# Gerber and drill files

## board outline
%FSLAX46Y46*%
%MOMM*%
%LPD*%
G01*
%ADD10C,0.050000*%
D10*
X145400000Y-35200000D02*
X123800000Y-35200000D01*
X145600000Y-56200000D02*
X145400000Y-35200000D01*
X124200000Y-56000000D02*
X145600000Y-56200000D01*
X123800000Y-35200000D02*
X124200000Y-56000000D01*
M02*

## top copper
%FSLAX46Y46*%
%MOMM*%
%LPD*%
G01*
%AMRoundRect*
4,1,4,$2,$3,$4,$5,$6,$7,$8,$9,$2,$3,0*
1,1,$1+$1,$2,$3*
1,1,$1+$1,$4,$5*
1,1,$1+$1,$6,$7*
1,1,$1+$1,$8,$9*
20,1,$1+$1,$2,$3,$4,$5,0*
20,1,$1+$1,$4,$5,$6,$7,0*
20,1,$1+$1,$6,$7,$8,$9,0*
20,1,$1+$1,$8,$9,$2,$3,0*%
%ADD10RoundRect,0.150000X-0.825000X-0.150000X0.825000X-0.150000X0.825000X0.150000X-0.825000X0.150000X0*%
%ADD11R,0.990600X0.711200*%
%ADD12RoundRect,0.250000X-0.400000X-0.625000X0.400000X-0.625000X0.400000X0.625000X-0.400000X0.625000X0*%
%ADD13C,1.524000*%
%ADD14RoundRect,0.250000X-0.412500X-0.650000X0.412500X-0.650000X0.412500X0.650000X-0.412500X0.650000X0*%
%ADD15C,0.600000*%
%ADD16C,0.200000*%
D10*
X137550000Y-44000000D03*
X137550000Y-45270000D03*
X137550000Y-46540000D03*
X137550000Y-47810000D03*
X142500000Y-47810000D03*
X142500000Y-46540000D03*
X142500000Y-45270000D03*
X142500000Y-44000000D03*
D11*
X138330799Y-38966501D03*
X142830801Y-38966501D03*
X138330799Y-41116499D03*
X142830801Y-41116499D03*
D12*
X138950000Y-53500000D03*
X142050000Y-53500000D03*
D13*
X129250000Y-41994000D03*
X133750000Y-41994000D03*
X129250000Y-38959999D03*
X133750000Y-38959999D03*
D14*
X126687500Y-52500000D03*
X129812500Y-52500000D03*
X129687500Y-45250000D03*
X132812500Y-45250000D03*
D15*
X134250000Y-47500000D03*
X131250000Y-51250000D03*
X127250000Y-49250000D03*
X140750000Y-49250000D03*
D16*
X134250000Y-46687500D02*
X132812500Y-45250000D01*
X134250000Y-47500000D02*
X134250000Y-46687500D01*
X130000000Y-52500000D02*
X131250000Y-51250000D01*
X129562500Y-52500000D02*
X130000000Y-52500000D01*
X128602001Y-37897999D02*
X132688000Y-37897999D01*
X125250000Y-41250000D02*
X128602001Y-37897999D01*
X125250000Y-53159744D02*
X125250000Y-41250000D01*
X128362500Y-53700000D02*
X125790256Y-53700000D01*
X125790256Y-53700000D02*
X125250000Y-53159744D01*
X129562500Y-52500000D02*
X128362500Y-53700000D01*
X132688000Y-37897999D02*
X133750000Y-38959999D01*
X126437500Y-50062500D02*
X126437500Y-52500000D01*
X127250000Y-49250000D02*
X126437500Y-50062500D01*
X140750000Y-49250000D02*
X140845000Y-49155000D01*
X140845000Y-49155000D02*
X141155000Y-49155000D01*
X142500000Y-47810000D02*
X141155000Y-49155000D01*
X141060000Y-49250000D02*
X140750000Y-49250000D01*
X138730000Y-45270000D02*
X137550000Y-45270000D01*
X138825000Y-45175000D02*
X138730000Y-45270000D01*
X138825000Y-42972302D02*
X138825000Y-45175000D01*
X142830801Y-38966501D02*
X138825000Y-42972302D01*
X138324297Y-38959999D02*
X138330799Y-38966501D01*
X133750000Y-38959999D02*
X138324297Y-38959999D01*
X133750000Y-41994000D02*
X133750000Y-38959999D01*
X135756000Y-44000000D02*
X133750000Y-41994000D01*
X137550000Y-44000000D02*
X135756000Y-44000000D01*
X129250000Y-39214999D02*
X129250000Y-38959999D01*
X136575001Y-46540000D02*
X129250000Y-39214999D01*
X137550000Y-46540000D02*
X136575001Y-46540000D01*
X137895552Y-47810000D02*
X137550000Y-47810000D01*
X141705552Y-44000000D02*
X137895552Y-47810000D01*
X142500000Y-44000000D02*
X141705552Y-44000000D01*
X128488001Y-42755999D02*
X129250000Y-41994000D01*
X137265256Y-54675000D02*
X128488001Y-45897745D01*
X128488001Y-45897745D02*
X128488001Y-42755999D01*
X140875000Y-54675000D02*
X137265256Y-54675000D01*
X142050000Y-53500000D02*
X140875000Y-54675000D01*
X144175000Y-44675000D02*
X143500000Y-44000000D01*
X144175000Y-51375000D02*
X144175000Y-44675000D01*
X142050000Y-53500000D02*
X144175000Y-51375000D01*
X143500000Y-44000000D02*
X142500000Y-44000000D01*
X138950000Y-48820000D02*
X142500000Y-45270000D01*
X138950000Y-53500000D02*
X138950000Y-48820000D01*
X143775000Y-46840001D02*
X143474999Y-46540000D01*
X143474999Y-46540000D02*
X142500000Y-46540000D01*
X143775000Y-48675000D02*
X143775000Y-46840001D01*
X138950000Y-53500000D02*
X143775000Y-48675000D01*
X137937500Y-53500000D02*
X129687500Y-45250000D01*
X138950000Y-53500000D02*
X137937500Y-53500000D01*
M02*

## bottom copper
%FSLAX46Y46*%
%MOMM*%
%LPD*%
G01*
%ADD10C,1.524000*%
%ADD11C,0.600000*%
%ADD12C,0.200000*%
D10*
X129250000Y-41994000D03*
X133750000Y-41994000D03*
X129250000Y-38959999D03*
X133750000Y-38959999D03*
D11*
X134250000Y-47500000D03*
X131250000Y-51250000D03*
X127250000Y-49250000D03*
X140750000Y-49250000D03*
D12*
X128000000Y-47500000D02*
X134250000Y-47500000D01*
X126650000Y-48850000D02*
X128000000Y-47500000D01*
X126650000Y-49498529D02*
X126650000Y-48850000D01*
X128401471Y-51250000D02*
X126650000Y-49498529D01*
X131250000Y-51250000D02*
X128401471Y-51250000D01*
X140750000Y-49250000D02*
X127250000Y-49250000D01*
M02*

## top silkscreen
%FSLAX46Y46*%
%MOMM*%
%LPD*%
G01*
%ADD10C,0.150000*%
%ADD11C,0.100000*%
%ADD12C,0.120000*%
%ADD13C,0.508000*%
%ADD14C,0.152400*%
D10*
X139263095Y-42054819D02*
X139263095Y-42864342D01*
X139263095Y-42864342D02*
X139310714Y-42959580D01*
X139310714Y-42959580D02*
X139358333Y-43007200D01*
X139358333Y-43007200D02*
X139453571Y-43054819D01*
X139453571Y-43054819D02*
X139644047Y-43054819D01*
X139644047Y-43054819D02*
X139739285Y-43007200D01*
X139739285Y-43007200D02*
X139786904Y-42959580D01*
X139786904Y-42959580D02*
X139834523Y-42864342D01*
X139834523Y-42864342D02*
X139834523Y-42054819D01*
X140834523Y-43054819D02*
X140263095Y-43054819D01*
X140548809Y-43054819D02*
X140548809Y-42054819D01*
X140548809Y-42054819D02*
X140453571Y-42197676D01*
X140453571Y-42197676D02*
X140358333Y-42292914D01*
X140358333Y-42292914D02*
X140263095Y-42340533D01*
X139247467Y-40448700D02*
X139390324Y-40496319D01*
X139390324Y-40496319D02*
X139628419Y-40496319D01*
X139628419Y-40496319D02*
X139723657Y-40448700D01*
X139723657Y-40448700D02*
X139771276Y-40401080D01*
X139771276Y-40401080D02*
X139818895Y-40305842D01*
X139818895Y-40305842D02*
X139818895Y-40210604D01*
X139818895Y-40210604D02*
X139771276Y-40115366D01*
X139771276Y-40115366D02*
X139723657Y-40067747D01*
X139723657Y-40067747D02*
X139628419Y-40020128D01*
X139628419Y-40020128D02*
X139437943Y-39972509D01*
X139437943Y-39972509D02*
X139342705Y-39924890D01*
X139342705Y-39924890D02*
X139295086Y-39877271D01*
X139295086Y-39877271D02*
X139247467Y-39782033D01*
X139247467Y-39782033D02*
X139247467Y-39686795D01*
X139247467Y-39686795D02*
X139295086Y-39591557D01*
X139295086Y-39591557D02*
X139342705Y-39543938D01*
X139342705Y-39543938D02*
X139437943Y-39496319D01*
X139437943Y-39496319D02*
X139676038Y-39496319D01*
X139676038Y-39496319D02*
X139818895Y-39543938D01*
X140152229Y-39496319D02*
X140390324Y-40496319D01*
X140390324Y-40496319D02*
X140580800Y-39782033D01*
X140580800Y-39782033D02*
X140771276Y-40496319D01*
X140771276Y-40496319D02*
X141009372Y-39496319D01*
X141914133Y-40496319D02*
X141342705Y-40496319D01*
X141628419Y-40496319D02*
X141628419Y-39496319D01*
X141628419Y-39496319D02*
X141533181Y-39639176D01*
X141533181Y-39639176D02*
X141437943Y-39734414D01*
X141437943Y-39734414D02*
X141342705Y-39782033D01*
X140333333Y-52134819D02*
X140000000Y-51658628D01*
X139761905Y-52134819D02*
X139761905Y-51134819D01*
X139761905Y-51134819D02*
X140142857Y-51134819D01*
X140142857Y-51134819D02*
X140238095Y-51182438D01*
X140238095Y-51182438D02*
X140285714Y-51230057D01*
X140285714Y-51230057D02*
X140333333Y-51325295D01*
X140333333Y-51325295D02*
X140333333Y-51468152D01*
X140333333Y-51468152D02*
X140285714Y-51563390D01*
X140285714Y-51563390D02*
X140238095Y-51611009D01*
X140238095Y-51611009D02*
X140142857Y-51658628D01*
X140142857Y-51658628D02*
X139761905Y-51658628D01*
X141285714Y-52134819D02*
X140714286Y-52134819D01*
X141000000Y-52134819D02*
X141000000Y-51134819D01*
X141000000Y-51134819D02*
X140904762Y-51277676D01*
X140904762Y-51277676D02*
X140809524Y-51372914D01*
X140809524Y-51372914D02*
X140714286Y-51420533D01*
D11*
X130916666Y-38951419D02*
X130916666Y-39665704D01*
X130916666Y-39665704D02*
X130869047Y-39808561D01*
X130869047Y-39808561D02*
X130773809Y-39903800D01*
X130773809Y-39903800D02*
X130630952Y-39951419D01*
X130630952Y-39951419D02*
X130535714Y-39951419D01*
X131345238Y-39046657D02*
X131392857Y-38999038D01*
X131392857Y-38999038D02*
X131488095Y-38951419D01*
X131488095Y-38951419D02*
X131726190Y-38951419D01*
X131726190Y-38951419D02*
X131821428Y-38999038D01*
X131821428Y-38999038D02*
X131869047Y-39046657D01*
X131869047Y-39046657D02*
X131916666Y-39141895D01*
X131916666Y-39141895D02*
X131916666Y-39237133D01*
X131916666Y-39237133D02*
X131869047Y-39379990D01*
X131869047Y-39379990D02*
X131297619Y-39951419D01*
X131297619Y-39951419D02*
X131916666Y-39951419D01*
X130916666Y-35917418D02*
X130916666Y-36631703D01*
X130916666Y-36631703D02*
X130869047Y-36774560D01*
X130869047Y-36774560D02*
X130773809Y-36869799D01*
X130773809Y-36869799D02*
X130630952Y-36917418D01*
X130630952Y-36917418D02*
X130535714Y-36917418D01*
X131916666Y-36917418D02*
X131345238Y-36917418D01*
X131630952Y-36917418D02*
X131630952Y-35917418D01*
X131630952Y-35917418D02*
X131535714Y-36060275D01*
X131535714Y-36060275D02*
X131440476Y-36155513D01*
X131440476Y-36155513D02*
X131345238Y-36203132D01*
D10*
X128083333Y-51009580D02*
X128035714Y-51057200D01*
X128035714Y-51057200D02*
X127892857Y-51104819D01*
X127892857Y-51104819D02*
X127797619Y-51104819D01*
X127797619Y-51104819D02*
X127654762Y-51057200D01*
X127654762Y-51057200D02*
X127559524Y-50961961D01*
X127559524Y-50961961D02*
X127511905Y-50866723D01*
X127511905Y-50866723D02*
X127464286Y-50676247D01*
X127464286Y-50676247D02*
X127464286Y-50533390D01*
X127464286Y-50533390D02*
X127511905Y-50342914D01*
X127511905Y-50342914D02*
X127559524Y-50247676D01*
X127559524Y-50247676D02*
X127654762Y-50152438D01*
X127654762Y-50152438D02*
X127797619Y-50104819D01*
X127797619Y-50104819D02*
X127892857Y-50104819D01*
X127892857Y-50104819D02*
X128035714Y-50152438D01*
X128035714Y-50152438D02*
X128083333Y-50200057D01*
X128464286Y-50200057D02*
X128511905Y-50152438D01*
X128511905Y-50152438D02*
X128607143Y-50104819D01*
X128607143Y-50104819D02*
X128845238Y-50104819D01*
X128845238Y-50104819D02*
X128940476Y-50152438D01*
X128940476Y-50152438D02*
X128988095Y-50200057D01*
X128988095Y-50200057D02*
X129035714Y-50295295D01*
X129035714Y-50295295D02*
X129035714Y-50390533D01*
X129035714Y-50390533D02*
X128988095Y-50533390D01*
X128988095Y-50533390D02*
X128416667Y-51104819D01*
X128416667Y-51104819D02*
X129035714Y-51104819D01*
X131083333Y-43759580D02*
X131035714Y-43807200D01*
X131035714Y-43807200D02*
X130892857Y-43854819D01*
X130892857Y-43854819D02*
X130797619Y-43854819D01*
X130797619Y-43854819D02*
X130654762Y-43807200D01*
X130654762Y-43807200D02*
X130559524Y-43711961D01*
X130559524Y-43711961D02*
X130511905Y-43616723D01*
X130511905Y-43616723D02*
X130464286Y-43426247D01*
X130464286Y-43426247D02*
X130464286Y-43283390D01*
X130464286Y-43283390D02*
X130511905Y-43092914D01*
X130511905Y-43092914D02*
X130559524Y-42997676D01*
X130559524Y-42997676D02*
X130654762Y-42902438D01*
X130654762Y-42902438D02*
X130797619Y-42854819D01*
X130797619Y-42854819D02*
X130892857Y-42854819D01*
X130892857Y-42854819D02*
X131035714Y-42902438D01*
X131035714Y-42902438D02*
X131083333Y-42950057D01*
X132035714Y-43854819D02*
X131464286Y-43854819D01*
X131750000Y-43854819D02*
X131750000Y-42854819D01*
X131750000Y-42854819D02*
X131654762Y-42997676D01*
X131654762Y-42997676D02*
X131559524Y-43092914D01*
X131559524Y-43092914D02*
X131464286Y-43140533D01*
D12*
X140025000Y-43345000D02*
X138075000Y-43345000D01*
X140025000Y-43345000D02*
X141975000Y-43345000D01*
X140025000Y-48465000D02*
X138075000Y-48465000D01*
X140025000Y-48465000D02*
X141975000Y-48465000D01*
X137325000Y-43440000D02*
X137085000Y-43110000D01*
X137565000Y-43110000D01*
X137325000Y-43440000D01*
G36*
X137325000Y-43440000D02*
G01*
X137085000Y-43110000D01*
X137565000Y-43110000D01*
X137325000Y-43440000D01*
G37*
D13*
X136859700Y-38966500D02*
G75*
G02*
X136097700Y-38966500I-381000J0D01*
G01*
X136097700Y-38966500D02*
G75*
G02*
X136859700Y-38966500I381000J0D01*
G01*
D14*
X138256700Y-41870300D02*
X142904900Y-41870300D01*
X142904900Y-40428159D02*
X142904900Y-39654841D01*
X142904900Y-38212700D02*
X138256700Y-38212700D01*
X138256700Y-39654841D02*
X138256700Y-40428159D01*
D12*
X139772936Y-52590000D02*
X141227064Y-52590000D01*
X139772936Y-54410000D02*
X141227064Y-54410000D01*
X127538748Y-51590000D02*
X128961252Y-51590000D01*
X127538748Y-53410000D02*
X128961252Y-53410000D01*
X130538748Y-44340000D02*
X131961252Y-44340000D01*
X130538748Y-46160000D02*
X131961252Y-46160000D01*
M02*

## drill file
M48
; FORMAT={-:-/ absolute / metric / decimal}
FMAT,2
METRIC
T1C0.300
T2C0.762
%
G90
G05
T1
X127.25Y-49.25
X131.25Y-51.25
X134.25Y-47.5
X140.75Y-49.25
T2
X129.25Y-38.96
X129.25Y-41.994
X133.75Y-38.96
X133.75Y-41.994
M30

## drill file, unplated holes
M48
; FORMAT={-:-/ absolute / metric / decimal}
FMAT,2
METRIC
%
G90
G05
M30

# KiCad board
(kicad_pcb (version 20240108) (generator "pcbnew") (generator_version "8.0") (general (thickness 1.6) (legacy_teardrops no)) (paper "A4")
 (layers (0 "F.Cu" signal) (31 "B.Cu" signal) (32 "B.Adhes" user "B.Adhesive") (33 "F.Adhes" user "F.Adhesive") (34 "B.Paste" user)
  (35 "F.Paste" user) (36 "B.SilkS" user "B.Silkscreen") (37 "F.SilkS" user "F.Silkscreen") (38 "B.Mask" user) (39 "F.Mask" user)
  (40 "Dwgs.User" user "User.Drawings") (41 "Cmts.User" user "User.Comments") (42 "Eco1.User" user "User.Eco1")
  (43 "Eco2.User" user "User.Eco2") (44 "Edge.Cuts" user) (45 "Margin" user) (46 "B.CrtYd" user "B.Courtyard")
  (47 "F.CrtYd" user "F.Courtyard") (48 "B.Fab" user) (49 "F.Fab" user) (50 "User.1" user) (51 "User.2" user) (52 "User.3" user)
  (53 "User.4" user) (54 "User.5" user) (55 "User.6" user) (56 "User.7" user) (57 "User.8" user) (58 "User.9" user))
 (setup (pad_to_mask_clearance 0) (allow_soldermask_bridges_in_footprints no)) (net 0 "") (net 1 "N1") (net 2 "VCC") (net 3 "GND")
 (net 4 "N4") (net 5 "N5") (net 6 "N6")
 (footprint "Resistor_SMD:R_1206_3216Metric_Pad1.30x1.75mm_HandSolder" (layer "F.Cu") (at 140.5 53.5)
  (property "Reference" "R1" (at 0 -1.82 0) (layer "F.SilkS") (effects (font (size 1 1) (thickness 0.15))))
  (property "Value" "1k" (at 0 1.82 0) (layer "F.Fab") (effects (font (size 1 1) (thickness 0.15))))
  (fp_line (start -0.727064 -0.91) (end 0.727064 -0.91) (stroke (width 0.12) (type solid)) (layer "F.SilkS"))
  (fp_line (start -0.727064 0.91) (end 0.727064 0.91) (stroke (width 0.12) (type solid)) (layer "F.SilkS"))
  (pad "1" smd roundrect (at -1.55 0) (size 1.3 1.75) (layers "F.Cu" "F.Paste" "F.Mask") (roundrect_rratio 0.192308) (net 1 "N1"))
  (pad "2" smd roundrect (at 1.55 0) (size 1.3 1.75) (layers "F.Cu" "F.Paste" "F.Mask") (roundrect_rratio 0.192308) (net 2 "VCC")))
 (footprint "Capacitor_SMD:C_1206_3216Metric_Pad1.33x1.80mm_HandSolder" (layer "F.Cu") (at 131.25 45.25)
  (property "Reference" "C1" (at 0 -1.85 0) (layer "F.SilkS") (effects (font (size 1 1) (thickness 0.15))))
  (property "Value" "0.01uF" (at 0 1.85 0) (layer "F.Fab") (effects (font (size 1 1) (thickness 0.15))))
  (fp_line (start -0.711252 -0.91) (end 0.711252 -0.91) (stroke (width 0.12) (type solid)) (layer "F.SilkS"))
  (fp_line (start -0.711252 0.91) (end 0.711252 0.91) (stroke (width 0.12) (type solid)) (layer "F.SilkS"))
  (pad "1" smd roundrect (at -1.5625 0) (size 1.325 1.8) (layers "F.Cu" "F.Paste" "F.Mask") (roundrect_rratio 0.188679) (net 1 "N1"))
  (pad "2" smd roundrect (at 1.5625 0) (size 1.325 1.8) (layers "F.Cu" "F.Paste" "F.Mask") (roundrect_rratio 0.188679) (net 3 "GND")))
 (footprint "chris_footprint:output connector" (layer "F.Cu") (at 131.25 36.959999)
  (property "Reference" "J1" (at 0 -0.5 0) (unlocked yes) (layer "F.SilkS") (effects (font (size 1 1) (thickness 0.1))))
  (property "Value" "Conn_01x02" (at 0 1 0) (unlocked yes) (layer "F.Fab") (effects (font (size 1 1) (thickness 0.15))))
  (pad "1" thru_hole circle (at -2 2) (size 1.524 1.524) (drill 0.762) (layers "*.Cu" "*.Mask") (remove_unused_layers no) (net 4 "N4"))
  (pad "2" thru_hole circle (at 2.5 2) (size 1.524 1.524) (drill 0.762) (layers "*.Cu" "*.Mask") (remove_unused_layers no) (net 3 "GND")))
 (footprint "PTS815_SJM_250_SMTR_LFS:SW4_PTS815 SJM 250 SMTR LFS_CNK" (layer "F.Cu") (at 140.5808 40.0415)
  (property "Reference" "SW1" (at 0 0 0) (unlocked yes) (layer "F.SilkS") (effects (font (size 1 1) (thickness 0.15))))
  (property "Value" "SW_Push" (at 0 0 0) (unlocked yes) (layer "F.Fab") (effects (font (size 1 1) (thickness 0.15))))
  (fp_line (start -2.3241 -0.386659) (end -2.3241 0.386659) (stroke (width 0.1524) (type solid)) (layer "F.SilkS"))
  (fp_line (start -2.3241 1.8288) (end 2.3241 1.8288) (stroke (width 0.1524) (type solid)) (layer "F.SilkS"))
  (fp_line (start 2.3241 -1.8288) (end -2.3241 -1.8288) (stroke (width 0.1524) (type solid)) (layer "F.SilkS"))
  (fp_line (start 2.3241 0.386659) (end 2.3241 -0.386659) (stroke (width 0.1524) (type solid)) (layer "F.SilkS"))
  (fp_circle (center -4.1021 -1.075) (end -3.7211 -1.075) (stroke (width 0.508) (type solid)) (fill none) (layer "F.SilkS"))
  (pad "1" smd rect (at -2.250001 -1.074999) (size 0.9906 0.7112) (layers "F.Cu" "F.Paste" "F.Mask") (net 3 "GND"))
  (pad "2" smd rect (at 2.250001 -1.074999) (size 0.9906 0.7112) (layers "F.Cu" "F.Paste" "F.Mask") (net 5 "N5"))
  (pad "3" smd rect (at -2.250001 1.074999) (size 0.9906 0.7112) (layers "F.Cu" "F.Paste" "F.Mask"))
  (pad "4" smd rect (at 2.250001 1.074999) (size 0.9906 0.7112) (layers "F.Cu" "F.Paste" "F.Mask")))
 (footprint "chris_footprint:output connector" (layer "F.Cu") (at 131.25 39.994)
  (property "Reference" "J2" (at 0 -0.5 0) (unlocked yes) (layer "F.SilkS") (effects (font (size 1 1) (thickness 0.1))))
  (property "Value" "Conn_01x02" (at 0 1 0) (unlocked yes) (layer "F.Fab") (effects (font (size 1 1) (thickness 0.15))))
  (pad "1" thru_hole circle (at -2 2) (size 1.524 1.524) (drill 0.762) (layers "*.Cu" "*.Mask") (remove_unused_layers no) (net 2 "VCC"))
  (pad "2" thru_hole circle (at 2.5 2) (size 1.524 1.524) (drill 0.762) (layers "*.Cu" "*.Mask") (remove_unused_layers no) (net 3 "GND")))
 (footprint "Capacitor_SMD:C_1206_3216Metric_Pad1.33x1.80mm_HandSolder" (layer "F.Cu") (at 128.25 52.5)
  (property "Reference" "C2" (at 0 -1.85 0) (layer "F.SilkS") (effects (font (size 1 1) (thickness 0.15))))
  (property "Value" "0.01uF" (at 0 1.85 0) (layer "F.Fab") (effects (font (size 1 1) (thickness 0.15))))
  (fp_line (start -0.711252 -0.91) (end 0.711252 -0.91) (stroke (width 0.12) (type solid)) (layer "F.SilkS"))
  (fp_line (start -0.711252 0.91) (end 0.711252 0.91) (stroke (width 0.12) (type solid)) (layer "F.SilkS"))
  (pad "1" smd roundrect (at -1.5625 0) (size 1.325 1.8) (layers "F.Cu" "F.Paste" "F.Mask") (roundrect_rratio 0.188679) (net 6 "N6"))
  (pad "2" smd roundrect (at 1.5625 0) (size 1.325 1.8) (layers "F.Cu" "F.Paste" "F.Mask") (roundrect_rratio 0.188679) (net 3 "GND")))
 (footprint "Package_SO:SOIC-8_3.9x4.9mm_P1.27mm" (layer "F.Cu") (at 140.025 45.905)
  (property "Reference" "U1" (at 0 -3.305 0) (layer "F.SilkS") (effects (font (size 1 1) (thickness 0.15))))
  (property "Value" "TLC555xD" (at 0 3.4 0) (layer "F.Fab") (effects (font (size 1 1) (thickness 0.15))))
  (fp_line (start 0 -2.56) (end -1.95 -2.56) (stroke (width 0.12) (type solid)) (layer "F.SilkS"))
  (fp_line (start 0 -2.56) (end 1.95 -2.56) (stroke (width 0.12) (type solid)) (layer "F.SilkS"))
  (fp_line (start 0 2.56) (end -1.95 2.56) (stroke (width 0.12) (type solid)) (layer "F.SilkS"))
  (fp_line (start 0 2.56) (end 1.95 2.56) (stroke (width 0.12) (type solid)) (layer "F.SilkS"))
  (fp_poly
   (pts (xy -2.7 -2.465) (xy -2.94 -2.795) (xy -2.46 -2.795) (xy -2.7 -2.465)) (stroke (width 0.12) (type solid)) (fill solid)
   (layer "F.SilkS"))
  (pad "1" smd roundrect (at -2.475 -1.905) (size 1.95 0.6) (layers "F.Cu" "F.Paste" "F.Mask") (roundrect_rratio 0.25) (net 3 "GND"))
  (pad "2" smd roundrect (at -2.475 -0.635) (size 1.95 0.6) (layers "F.Cu" "F.Paste" "F.Mask") (roundrect_rratio 0.25) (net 5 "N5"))
  (pad "3" smd roundrect (at -2.475 0.635) (size 1.95 0.6) (layers "F.Cu" "F.Paste" "F.Mask") (roundrect_rratio 0.25) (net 4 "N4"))
  (pad "4" smd roundrect (at -2.475 1.905) (size 1.95 0.6) (layers "F.Cu" "F.Paste" "F.Mask") (roundrect_rratio 0.25) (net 2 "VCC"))
  (pad "5" smd roundrect (at 2.475 1.905) (size 1.95 0.6) (layers "F.Cu" "F.Paste" "F.Mask") (roundrect_rratio 0.25) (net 6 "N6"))
  (pad "6" smd roundrect (at 2.475 0.635) (size 1.95 0.6) (layers "F.Cu" "F.Paste" "F.Mask") (roundrect_rratio 0.25) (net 1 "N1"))
  (pad "7" smd roundrect (at 2.475 -0.635) (size 1.95 0.6) (layers "F.Cu" "F.Paste" "F.Mask") (roundrect_rratio 0.25) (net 1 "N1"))
  (pad "8" smd roundrect (at 2.475 -1.905) (size 1.95 0.6) (layers "F.Cu" "F.Paste" "F.Mask") (roundrect_rratio 0.25) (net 2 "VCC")))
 (gr_line (start 123.8 35.2) (end 124.2 56) (stroke (width 0.05) (type default)) (layer "Edge.Cuts"))
 (gr_line (start 124.2 56) (end 145.6 56.2) (stroke (width 0.05) (type default)) (layer "Edge.Cuts"))
 (gr_line (start 145.6 56.2) (end 145.4 35.2) (stroke (width 0.05) (type default)) (layer "Edge.Cuts"))
 (gr_line (start 145.4 35.2) (end 123.8 35.2) (stroke (width 0.05) (type default)) (layer "Edge.Cuts"))
 (segment (start 128.3625 53.7) (end 125.790256 53.7) (width 0.2) (layer "F.Cu") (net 3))
 (segment (start 133.75 38.959999) (end 138.324297 38.959999) (width 0.2) (layer "F.Cu") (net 3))
 (segment (start 138.324297 38.959999) (end 138.330799 38.966501) (width 0.2) (layer "F.Cu") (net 3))
 (segment (start 134.25 47.5) (end 134.25 46.6875) (width 0.2) (layer "F.Cu") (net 3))
 (segment (start 132.688 37.897999) (end 133.75 38.959999) (width 0.2) (layer "F.Cu") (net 3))
 (segment (start 129.5625 52.5) (end 128.3625 53.7) (width 0.2) (layer "F.Cu") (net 3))
 (segment (start 128.602001 37.897999) (end 132.688 37.897999) (width 0.2) (layer "F.Cu") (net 3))
 (segment (start 133.75 41.994) (end 133.75 38.959999) (width 0.2) (layer "F.Cu") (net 3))
 (segment (start 134.25 46.6875) (end 132.8125 45.25) (width 0.2) (layer "F.Cu") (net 3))
 (segment (start 135.756 44) (end 133.75 41.994) (width 0.2) (layer "F.Cu") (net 3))
 (segment (start 137.55 44) (end 135.756 44) (width 0.2) (layer "F.Cu") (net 3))
 (segment (start 129.5625 52.5) (end 130 52.5) (width 0.2) (layer "F.Cu") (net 3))
 (segment (start 125.25 53.159744) (end 125.25 41.25) (width 0.2) (layer "F.Cu") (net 3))
 (segment (start 125.25 41.25) (end 128.602001 37.897999) (width 0.2) (layer "F.Cu") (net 3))
 (segment (start 125.790256 53.7) (end 125.25 53.159744) (width 0.2) (layer "F.Cu") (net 3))
 (segment (start 130 52.5) (end 131.25 51.25) (width 0.2) (layer "F.Cu") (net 3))
 (via (at 134.25 47.5) (size 0.6) (drill 0.3) (layers "F.Cu" "B.Cu") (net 3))
 (via (at 131.25 51.25) (size 0.6) (drill 0.3) (layers "F.Cu" "B.Cu") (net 3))
 (segment (start 128.401471 51.25) (end 126.65 49.498529) (width 0.2) (layer "B.Cu") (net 3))
 (segment (start 126.65 49.498529) (end 126.65 48.85) (width 0.2) (layer "B.Cu") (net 3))
 (segment (start 128 47.5) (end 134.25 47.5) (width 0.2) (layer "B.Cu") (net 3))
 (segment (start 126.65 48.85) (end 128 47.5) (width 0.2) (layer "B.Cu") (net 3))
 (segment (start 131.25 51.25) (end 128.401471 51.25) (width 0.2) (layer "B.Cu") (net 3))
 (segment (start 143.775 48.675) (end 143.775 46.840001) (width 0.2) (layer "F.Cu") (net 1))
 (segment (start 143.474999 46.54) (end 142.5 46.54) (width 0.2) (layer "F.Cu") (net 1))
 (segment (start 138.95 53.5) (end 143.775 48.675) (width 0.2) (layer "F.Cu") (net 1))
 (segment (start 138.95 53.5) (end 138.95 48.82) (width 0.2) (layer "F.Cu") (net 1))
 (segment (start 138.95 48.82) (end 142.5 45.27) (width 0.2) (layer "F.Cu") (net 1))
 (segment (start 137.9375 53.5) (end 129.6875 45.25) (width 0.2) (layer "F.Cu") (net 1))
 (segment (start 138.95 53.5) (end 137.9375 53.5) (width 0.2) (layer "F.Cu") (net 1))
 (segment (start 143.775 46.840001) (end 143.474999 46.54) (width 0.2) (layer "F.Cu") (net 1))
 (segment (start 141.06 49.25) (end 140.75 49.25) (width 0.2) (layer "F.Cu") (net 6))
 (segment (start 126.4375 50.0625) (end 126.4375 52.5) (width 0.2) (layer "F.Cu") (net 6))
 (segment (start 142.5 47.81) (end 141.155 49.155) (width 0.2) (layer "F.Cu") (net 6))
 (segment (start 127.25 49.25) (end 126.4375 50.0625) (width 0.2) (layer "F.Cu") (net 6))
 (segment (start 140.75 49.25) (end 140.845 49.155) (width 0.2) (layer "F.Cu") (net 6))
 (segment (start 140.845 49.155) (end 141.155 49.155) (width 0.2) (layer "F.Cu") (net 6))
 (via (at 140.75 49.25) (size 0.6) (drill 0.3) (layers "F.Cu" "B.Cu") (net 6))
 (via (at 127.25 49.25) (size 0.6) (drill 0.3) (layers "F.Cu" "B.Cu") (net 6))
 (segment (start 140.75 49.25) (end 127.25 49.25) (width 0.2) (layer "B.Cu") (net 6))
 (segment (start 136.575001 46.54) (end 129.25 39.214999) (width 0.2) (layer "F.Cu") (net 4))
 (segment (start 129.25 39.214999) (end 129.25 38.959999) (width 0.2) (layer "F.Cu") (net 4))
 (segment (start 137.55 46.54) (end 136.575001 46.54) (width 0.2) (layer "F.Cu") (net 4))
 (segment (start 142.05 53.5) (end 144.175 51.375) (width 0.2) (layer "F.Cu") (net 2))
 (segment (start 141.705552 44) (end 137.895552 47.81) (width 0.2) (layer "F.Cu") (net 2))
 (segment (start 137.265256 54.675) (end 128.488001 45.897745) (width 0.2) (layer "F.Cu") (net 2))
 (segment (start 128.488001 42.755999) (end 129.25 41.994) (width 0.2) (layer "F.Cu") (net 2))
 (segment (start 144.175 44.675) (end 143.5 44) (width 0.2) (layer "F.Cu") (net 2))
 (segment (start 140.875 54.675) (end 137.265256 54.675) (width 0.2) (layer "F.Cu") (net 2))
 (segment (start 142.05 53.5) (end 140.875 54.675) (width 0.2) (layer "F.Cu") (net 2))
 (segment (start 128.488001 45.897745) (end 128.488001 42.755999) (width 0.2) (layer "F.Cu") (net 2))
 (segment (start 143.5 44) (end 142.5 44) (width 0.2) (layer "F.Cu") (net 2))
 (segment (start 137.895552 47.81) (end 137.55 47.81) (width 0.2) (layer "F.Cu") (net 2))
 (segment (start 142.5 44) (end 141.705552 44) (width 0.2) (layer "F.Cu") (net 2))
 (segment (start 144.175 51.375) (end 144.175 44.675) (width 0.2) (layer "F.Cu") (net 2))
 (segment (start 142.830801 38.966501) (end 138.825 42.972302) (width 0.2) (layer "F.Cu") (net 5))
 (segment (start 138.825 45.175) (end 138.73 45.27) (width 0.2) (layer "F.Cu") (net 5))
 (segment (start 138.825 42.972302) (end 138.825 45.175) (width 0.2) (layer "F.Cu") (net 5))
 (segment (start 138.73 45.27) (end 137.55 45.27) (width 0.2) (layer "F.Cu") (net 5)))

